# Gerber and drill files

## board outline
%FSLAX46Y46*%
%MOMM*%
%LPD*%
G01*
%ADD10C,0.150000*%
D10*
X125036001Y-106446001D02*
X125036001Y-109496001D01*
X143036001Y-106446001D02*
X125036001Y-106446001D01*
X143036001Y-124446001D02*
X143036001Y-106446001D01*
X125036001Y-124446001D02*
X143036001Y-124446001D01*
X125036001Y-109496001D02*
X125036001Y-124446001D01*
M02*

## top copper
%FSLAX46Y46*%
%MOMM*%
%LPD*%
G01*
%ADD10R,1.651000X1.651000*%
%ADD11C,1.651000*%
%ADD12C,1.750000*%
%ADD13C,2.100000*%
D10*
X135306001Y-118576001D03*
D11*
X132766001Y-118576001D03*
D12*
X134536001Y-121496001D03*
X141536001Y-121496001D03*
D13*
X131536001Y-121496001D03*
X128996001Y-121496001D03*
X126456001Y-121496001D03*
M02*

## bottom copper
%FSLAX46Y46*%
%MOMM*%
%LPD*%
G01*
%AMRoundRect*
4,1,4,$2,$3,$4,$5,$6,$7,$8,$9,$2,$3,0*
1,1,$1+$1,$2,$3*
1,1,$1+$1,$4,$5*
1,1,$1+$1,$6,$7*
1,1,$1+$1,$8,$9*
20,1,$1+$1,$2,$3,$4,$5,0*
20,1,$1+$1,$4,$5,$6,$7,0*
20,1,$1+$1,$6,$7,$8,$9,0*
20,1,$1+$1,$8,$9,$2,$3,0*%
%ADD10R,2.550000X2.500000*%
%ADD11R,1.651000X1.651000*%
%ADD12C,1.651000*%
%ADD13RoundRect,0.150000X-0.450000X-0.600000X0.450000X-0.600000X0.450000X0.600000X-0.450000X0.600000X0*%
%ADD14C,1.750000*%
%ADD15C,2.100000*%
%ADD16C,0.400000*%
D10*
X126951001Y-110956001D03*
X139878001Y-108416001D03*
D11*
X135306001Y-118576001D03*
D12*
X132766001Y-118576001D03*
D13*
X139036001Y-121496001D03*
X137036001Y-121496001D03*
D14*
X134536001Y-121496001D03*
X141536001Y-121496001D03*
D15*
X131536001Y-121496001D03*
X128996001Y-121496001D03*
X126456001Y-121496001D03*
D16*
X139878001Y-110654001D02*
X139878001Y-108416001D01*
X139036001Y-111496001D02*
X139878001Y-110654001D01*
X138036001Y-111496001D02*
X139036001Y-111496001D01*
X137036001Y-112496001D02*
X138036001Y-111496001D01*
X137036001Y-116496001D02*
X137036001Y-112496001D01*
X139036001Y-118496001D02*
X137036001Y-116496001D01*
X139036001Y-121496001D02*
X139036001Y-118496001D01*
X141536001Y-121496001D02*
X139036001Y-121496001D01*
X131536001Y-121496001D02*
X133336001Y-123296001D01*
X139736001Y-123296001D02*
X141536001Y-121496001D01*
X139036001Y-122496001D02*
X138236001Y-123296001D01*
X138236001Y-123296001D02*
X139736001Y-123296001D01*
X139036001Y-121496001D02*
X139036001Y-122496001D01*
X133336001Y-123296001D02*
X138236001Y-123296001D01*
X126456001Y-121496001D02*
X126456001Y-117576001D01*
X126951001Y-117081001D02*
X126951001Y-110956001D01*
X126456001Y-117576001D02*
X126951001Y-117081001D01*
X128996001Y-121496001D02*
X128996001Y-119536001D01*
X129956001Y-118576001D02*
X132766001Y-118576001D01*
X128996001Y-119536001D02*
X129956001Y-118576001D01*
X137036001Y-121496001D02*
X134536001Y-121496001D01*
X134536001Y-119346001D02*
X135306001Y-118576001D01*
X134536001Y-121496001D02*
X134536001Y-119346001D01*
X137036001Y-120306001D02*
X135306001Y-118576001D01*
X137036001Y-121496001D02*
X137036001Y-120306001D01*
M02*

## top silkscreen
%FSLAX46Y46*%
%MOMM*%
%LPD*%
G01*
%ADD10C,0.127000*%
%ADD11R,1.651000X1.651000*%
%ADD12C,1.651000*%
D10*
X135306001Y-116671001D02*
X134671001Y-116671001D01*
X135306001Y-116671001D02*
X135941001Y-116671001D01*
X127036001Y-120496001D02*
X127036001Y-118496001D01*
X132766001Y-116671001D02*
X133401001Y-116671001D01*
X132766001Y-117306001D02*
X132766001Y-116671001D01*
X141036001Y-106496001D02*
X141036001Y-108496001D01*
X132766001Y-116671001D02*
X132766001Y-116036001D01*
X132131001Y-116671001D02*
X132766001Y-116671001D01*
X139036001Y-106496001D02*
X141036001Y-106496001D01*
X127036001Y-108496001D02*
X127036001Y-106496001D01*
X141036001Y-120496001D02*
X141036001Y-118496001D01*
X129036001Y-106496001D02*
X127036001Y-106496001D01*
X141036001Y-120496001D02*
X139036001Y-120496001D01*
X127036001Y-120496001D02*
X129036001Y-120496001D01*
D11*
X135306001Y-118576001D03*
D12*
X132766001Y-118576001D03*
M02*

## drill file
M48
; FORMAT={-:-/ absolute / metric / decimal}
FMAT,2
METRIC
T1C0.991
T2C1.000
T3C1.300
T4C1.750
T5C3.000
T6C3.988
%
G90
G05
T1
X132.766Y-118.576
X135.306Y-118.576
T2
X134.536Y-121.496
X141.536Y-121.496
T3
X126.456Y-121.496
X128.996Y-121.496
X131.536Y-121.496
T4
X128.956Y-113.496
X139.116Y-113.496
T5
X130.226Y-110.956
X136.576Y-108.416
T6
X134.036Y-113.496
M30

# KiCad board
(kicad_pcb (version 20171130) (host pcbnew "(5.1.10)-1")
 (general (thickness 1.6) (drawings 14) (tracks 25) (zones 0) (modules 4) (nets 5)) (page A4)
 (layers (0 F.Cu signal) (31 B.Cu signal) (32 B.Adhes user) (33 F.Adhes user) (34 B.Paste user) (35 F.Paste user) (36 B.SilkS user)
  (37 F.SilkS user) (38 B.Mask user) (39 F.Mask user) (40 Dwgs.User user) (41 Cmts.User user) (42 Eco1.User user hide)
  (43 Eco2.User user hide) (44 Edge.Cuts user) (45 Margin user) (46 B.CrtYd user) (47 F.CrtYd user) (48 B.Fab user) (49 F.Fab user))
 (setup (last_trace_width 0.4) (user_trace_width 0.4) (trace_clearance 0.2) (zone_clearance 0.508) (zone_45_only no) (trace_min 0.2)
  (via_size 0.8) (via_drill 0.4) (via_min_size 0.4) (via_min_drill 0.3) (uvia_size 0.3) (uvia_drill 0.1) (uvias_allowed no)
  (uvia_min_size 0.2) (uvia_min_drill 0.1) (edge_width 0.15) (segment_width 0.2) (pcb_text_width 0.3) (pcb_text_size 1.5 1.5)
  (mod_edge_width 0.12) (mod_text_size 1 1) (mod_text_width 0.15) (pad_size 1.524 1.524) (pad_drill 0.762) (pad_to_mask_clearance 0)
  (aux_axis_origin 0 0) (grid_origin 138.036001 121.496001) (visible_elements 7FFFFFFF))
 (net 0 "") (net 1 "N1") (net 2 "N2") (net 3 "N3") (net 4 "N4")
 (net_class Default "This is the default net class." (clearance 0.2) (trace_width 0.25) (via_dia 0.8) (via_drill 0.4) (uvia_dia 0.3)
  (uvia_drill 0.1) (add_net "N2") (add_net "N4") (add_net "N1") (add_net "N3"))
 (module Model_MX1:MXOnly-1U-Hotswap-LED (layer F.Cu) (at 134.036001 113.496001)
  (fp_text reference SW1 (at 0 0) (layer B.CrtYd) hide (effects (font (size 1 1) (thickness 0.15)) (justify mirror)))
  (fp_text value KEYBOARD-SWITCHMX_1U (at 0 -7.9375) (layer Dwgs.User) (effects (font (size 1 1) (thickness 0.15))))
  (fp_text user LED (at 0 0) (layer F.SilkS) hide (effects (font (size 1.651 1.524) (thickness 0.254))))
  (fp_line (start 1.27 3.175) (end 0.635 3.175) (layer F.SilkS) (width 0.127))
  (fp_line (start 1.27 3.175) (end 1.905 3.175) (layer F.SilkS) (width 0.127))
  (fp_line (start -7 7) (end -7 5) (layer F.SilkS) (width 0.127))
  (fp_line (start -1.27 3.175) (end -0.635 3.175) (layer F.SilkS) (width 0.127))
  (fp_line (start -1.27 3.81) (end -1.27 3.175) (layer F.SilkS) (width 0.127))
  (fp_line (start 7 -7) (end 7 -5) (layer F.SilkS) (width 0.127))
  (fp_line (start -1.27 3.175) (end -1.27 2.54) (layer F.SilkS) (width 0.127))
  (fp_line (start -1.905 3.175) (end -1.27 3.175) (layer F.SilkS) (width 0.127))
  (fp_line (start 5 -7) (end 7 -7) (layer F.SilkS) (width 0.127))
  (fp_line (start -7 -5) (end -7 -7) (layer F.SilkS) (width 0.127))
  (fp_line (start 7 7) (end 7 5) (layer F.SilkS) (width 0.127))
  (fp_line (start -5 -7) (end -7 -7) (layer F.SilkS) (width 0.127))
  (fp_line (start 7 7) (end 5 7) (layer F.SilkS) (width 0.127))
  (fp_line (start -7 7) (end -5 7) (layer F.SilkS) (width 0.127))
  (pad "" np_thru_hole circle (at 2.54 -5.08) (size 3 3) (drill 3) (layers *.Cu *.Mask))
  (pad "" np_thru_hole circle (at 0 0) (size 3.9878 3.9878) (drill 3.9878) (layers *.Cu *.Mask))
  (pad "" np_thru_hole circle (at -3.81 -2.54) (size 3 3) (drill 3) (layers *.Cu *.Mask))
  (pad "" np_thru_hole circle (at -5.08 0 48.0996) (size 1.75 1.75) (drill 1.75) (layers *.Cu *.Mask))
  (pad "" np_thru_hole circle (at 5.08 0 48.0996) (size 1.75 1.75) (drill 1.75) (layers *.Cu *.Mask))
  (pad S1 smd rect (at -7.085 -2.54) (size 2.55 2.5) (layers B.Cu B.Paste B.Mask) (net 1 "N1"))
  (pad S2 smd rect (at 5.842 -5.08) (size 2.55 2.5) (layers B.Cu B.Paste B.Mask) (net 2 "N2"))
  (pad C thru_hole rect (at 1.27 5.08) (size 1.651 1.651) (drill 0.9906) (layers *.Cu *.SilkS *.Mask) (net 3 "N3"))
  (pad A thru_hole circle (at -1.27 5.08) (size 1.651 1.651) (drill 0.9906) (layers *.Cu *.SilkS *.Mask) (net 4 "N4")))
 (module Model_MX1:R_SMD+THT (layer B.Cu) (at 138.036001 121.496001)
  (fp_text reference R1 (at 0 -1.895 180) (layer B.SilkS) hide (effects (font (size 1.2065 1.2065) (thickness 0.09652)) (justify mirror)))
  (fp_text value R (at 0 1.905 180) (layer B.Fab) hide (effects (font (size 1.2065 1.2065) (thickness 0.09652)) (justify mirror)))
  (pad 2 smd roundrect (at 1 0) (size 1.2 1.5) (layers B.Cu B.Paste B.Mask) (roundrect_rratio 0.125) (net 2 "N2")
   (solder_mask_margin 0.1016))
  (pad 1 smd roundrect (at -1 0) (size 1.2 1.5) (layers B.Cu B.Paste B.Mask) (roundrect_rratio 0.125) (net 3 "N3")
   (solder_mask_margin 0.1016))
  (pad 1 thru_hole circle (at -3.5 0) (size 1.75 1.75) (drill 1) (layers *.Cu *.Mask) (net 3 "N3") (solder_mask_margin 0.1016))
  (pad 2 thru_hole circle (at 3.5 0) (size 1.75 1.75) (drill 1) (layers *.Cu *.Mask) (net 2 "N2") (solder_mask_margin 0.1016)))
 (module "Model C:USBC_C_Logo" (layer B.Cu) (at 139.306001 117.576001 180)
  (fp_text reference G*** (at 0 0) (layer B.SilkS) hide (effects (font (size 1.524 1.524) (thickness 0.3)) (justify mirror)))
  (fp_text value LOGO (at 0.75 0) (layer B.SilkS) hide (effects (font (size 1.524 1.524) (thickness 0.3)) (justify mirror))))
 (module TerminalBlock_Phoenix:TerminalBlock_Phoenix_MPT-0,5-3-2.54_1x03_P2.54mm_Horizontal (layer B.Cu) (at 131.536001 121.496001 180)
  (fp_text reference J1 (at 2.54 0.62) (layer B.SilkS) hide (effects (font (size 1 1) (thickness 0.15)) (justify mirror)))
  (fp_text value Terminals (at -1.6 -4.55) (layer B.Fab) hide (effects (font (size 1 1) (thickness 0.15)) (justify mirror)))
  (pad 1 thru_hole circle (at 0 0 180) (size 2.1 2.1) (drill 1.3) (layers *.Cu *.Mask) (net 2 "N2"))
  (pad 2 thru_hole circle (at 2.54 0 180) (size 2.1 2.1) (drill 1.3) (layers *.Cu *.Mask) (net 4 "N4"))
  (pad 3 thru_hole circle (at 5.08 0 180) (size 2.1 2.1) (drill 1.3) (layers *.Cu *.Mask) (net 1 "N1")))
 (gr_line (start 125.036001 106.446001) (end 125.036001 109.496001) (layer Edge.Cuts) (width 0.15))
 (gr_line (start 143.036001 106.446001) (end 125.036001 106.446001) (layer Edge.Cuts) (width 0.15))
 (gr_line (start 143.036001 124.446001) (end 143.036001 106.446001) (layer Edge.Cuts) (width 0.15))
 (gr_line (start 125.036001 124.446001) (end 143.036001 124.446001) (layer Edge.Cuts) (width 0.15))
 (gr_line (start 125.036001 109.496001) (end 125.036001 124.446001) (layer Edge.Cuts) (width 0.15))
 (segment (start 139.878001 110.654001) (end 139.878001 108.416001) (width 0.4) (layer B.Cu) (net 2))
 (segment (start 139.036001 111.496001) (end 139.878001 110.654001) (width 0.4) (layer B.Cu) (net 2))
 (segment (start 138.036001 111.496001) (end 139.036001 111.496001) (width 0.4) (layer B.Cu) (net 2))
 (segment (start 137.036001 112.496001) (end 138.036001 111.496001) (width 0.4) (layer B.Cu) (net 2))
 (segment (start 137.036001 116.496001) (end 137.036001 112.496001) (width 0.4) (layer B.Cu) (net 2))
 (segment (start 139.036001 118.496001) (end 137.036001 116.496001) (width 0.4) (layer B.Cu) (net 2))
 (segment (start 139.036001 121.496001) (end 139.036001 118.496001) (width 0.4) (layer B.Cu) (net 2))
 (segment (start 141.536001 121.496001) (end 139.036001 121.496001) (width 0.4) (layer B.Cu) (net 2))
 (segment (start 131.536001 121.496001) (end 133.336001 123.296001) (width 0.4) (layer B.Cu) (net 2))
 (segment (start 139.736001 123.296001) (end 141.536001 121.496001) (width 0.4) (layer B.Cu) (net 2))
 (segment (start 139.036001 122.496001) (end 138.236001 123.296001) (width 0.4) (layer B.Cu) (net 2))
 (segment (start 138.236001 123.296001) (end 139.736001 123.296001) (width 0.4) (layer B.Cu) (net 2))
 (segment (start 139.036001 121.496001) (end 139.036001 122.496001) (width 0.4) (layer B.Cu) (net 2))
 (segment (start 133.336001 123.296001) (end 138.236001 123.296001) (width 0.4) (layer B.Cu) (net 2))
 (segment (start 126.456001 121.496001) (end 126.456001 117.576001) (width 0.4) (layer B.Cu) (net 1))
 (segment (start 126.951001 117.081001) (end 126.951001 110.956001) (width 0.4) (layer B.Cu) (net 1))
 (segment (start 126.456001 117.576001) (end 126.951001 117.081001) (width 0.4) (layer B.Cu) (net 1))
 (segment (start 128.996001 121.496001) (end 128.996001 119.536001) (width 0.4) (layer B.Cu) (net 4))
 (segment (start 129.956001 118.576001) (end 132.766001 118.576001) (width 0.4) (layer B.Cu) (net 4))
 (segment (start 128.996001 119.536001) (end 129.956001 118.576001) (width 0.4) (layer B.Cu) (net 4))
 (segment (start 137.036001 121.496001) (end 134.536001 121.496001) (width 0.4) (layer B.Cu) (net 3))
 (segment (start 134.536001 119.346001) (end 135.306001 118.576001) (width 0.4) (layer B.Cu) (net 3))
 (segment (start 134.536001 121.496001) (end 134.536001 119.346001) (width 0.4) (layer B.Cu) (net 3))
 (segment (start 137.036001 120.306001) (end 135.306001 118.576001) (width 0.4) (layer B.Cu) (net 3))
 (segment (start 137.036001 121.496001) (end 137.036001 120.306001) (width 0.4) (layer B.Cu) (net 3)))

